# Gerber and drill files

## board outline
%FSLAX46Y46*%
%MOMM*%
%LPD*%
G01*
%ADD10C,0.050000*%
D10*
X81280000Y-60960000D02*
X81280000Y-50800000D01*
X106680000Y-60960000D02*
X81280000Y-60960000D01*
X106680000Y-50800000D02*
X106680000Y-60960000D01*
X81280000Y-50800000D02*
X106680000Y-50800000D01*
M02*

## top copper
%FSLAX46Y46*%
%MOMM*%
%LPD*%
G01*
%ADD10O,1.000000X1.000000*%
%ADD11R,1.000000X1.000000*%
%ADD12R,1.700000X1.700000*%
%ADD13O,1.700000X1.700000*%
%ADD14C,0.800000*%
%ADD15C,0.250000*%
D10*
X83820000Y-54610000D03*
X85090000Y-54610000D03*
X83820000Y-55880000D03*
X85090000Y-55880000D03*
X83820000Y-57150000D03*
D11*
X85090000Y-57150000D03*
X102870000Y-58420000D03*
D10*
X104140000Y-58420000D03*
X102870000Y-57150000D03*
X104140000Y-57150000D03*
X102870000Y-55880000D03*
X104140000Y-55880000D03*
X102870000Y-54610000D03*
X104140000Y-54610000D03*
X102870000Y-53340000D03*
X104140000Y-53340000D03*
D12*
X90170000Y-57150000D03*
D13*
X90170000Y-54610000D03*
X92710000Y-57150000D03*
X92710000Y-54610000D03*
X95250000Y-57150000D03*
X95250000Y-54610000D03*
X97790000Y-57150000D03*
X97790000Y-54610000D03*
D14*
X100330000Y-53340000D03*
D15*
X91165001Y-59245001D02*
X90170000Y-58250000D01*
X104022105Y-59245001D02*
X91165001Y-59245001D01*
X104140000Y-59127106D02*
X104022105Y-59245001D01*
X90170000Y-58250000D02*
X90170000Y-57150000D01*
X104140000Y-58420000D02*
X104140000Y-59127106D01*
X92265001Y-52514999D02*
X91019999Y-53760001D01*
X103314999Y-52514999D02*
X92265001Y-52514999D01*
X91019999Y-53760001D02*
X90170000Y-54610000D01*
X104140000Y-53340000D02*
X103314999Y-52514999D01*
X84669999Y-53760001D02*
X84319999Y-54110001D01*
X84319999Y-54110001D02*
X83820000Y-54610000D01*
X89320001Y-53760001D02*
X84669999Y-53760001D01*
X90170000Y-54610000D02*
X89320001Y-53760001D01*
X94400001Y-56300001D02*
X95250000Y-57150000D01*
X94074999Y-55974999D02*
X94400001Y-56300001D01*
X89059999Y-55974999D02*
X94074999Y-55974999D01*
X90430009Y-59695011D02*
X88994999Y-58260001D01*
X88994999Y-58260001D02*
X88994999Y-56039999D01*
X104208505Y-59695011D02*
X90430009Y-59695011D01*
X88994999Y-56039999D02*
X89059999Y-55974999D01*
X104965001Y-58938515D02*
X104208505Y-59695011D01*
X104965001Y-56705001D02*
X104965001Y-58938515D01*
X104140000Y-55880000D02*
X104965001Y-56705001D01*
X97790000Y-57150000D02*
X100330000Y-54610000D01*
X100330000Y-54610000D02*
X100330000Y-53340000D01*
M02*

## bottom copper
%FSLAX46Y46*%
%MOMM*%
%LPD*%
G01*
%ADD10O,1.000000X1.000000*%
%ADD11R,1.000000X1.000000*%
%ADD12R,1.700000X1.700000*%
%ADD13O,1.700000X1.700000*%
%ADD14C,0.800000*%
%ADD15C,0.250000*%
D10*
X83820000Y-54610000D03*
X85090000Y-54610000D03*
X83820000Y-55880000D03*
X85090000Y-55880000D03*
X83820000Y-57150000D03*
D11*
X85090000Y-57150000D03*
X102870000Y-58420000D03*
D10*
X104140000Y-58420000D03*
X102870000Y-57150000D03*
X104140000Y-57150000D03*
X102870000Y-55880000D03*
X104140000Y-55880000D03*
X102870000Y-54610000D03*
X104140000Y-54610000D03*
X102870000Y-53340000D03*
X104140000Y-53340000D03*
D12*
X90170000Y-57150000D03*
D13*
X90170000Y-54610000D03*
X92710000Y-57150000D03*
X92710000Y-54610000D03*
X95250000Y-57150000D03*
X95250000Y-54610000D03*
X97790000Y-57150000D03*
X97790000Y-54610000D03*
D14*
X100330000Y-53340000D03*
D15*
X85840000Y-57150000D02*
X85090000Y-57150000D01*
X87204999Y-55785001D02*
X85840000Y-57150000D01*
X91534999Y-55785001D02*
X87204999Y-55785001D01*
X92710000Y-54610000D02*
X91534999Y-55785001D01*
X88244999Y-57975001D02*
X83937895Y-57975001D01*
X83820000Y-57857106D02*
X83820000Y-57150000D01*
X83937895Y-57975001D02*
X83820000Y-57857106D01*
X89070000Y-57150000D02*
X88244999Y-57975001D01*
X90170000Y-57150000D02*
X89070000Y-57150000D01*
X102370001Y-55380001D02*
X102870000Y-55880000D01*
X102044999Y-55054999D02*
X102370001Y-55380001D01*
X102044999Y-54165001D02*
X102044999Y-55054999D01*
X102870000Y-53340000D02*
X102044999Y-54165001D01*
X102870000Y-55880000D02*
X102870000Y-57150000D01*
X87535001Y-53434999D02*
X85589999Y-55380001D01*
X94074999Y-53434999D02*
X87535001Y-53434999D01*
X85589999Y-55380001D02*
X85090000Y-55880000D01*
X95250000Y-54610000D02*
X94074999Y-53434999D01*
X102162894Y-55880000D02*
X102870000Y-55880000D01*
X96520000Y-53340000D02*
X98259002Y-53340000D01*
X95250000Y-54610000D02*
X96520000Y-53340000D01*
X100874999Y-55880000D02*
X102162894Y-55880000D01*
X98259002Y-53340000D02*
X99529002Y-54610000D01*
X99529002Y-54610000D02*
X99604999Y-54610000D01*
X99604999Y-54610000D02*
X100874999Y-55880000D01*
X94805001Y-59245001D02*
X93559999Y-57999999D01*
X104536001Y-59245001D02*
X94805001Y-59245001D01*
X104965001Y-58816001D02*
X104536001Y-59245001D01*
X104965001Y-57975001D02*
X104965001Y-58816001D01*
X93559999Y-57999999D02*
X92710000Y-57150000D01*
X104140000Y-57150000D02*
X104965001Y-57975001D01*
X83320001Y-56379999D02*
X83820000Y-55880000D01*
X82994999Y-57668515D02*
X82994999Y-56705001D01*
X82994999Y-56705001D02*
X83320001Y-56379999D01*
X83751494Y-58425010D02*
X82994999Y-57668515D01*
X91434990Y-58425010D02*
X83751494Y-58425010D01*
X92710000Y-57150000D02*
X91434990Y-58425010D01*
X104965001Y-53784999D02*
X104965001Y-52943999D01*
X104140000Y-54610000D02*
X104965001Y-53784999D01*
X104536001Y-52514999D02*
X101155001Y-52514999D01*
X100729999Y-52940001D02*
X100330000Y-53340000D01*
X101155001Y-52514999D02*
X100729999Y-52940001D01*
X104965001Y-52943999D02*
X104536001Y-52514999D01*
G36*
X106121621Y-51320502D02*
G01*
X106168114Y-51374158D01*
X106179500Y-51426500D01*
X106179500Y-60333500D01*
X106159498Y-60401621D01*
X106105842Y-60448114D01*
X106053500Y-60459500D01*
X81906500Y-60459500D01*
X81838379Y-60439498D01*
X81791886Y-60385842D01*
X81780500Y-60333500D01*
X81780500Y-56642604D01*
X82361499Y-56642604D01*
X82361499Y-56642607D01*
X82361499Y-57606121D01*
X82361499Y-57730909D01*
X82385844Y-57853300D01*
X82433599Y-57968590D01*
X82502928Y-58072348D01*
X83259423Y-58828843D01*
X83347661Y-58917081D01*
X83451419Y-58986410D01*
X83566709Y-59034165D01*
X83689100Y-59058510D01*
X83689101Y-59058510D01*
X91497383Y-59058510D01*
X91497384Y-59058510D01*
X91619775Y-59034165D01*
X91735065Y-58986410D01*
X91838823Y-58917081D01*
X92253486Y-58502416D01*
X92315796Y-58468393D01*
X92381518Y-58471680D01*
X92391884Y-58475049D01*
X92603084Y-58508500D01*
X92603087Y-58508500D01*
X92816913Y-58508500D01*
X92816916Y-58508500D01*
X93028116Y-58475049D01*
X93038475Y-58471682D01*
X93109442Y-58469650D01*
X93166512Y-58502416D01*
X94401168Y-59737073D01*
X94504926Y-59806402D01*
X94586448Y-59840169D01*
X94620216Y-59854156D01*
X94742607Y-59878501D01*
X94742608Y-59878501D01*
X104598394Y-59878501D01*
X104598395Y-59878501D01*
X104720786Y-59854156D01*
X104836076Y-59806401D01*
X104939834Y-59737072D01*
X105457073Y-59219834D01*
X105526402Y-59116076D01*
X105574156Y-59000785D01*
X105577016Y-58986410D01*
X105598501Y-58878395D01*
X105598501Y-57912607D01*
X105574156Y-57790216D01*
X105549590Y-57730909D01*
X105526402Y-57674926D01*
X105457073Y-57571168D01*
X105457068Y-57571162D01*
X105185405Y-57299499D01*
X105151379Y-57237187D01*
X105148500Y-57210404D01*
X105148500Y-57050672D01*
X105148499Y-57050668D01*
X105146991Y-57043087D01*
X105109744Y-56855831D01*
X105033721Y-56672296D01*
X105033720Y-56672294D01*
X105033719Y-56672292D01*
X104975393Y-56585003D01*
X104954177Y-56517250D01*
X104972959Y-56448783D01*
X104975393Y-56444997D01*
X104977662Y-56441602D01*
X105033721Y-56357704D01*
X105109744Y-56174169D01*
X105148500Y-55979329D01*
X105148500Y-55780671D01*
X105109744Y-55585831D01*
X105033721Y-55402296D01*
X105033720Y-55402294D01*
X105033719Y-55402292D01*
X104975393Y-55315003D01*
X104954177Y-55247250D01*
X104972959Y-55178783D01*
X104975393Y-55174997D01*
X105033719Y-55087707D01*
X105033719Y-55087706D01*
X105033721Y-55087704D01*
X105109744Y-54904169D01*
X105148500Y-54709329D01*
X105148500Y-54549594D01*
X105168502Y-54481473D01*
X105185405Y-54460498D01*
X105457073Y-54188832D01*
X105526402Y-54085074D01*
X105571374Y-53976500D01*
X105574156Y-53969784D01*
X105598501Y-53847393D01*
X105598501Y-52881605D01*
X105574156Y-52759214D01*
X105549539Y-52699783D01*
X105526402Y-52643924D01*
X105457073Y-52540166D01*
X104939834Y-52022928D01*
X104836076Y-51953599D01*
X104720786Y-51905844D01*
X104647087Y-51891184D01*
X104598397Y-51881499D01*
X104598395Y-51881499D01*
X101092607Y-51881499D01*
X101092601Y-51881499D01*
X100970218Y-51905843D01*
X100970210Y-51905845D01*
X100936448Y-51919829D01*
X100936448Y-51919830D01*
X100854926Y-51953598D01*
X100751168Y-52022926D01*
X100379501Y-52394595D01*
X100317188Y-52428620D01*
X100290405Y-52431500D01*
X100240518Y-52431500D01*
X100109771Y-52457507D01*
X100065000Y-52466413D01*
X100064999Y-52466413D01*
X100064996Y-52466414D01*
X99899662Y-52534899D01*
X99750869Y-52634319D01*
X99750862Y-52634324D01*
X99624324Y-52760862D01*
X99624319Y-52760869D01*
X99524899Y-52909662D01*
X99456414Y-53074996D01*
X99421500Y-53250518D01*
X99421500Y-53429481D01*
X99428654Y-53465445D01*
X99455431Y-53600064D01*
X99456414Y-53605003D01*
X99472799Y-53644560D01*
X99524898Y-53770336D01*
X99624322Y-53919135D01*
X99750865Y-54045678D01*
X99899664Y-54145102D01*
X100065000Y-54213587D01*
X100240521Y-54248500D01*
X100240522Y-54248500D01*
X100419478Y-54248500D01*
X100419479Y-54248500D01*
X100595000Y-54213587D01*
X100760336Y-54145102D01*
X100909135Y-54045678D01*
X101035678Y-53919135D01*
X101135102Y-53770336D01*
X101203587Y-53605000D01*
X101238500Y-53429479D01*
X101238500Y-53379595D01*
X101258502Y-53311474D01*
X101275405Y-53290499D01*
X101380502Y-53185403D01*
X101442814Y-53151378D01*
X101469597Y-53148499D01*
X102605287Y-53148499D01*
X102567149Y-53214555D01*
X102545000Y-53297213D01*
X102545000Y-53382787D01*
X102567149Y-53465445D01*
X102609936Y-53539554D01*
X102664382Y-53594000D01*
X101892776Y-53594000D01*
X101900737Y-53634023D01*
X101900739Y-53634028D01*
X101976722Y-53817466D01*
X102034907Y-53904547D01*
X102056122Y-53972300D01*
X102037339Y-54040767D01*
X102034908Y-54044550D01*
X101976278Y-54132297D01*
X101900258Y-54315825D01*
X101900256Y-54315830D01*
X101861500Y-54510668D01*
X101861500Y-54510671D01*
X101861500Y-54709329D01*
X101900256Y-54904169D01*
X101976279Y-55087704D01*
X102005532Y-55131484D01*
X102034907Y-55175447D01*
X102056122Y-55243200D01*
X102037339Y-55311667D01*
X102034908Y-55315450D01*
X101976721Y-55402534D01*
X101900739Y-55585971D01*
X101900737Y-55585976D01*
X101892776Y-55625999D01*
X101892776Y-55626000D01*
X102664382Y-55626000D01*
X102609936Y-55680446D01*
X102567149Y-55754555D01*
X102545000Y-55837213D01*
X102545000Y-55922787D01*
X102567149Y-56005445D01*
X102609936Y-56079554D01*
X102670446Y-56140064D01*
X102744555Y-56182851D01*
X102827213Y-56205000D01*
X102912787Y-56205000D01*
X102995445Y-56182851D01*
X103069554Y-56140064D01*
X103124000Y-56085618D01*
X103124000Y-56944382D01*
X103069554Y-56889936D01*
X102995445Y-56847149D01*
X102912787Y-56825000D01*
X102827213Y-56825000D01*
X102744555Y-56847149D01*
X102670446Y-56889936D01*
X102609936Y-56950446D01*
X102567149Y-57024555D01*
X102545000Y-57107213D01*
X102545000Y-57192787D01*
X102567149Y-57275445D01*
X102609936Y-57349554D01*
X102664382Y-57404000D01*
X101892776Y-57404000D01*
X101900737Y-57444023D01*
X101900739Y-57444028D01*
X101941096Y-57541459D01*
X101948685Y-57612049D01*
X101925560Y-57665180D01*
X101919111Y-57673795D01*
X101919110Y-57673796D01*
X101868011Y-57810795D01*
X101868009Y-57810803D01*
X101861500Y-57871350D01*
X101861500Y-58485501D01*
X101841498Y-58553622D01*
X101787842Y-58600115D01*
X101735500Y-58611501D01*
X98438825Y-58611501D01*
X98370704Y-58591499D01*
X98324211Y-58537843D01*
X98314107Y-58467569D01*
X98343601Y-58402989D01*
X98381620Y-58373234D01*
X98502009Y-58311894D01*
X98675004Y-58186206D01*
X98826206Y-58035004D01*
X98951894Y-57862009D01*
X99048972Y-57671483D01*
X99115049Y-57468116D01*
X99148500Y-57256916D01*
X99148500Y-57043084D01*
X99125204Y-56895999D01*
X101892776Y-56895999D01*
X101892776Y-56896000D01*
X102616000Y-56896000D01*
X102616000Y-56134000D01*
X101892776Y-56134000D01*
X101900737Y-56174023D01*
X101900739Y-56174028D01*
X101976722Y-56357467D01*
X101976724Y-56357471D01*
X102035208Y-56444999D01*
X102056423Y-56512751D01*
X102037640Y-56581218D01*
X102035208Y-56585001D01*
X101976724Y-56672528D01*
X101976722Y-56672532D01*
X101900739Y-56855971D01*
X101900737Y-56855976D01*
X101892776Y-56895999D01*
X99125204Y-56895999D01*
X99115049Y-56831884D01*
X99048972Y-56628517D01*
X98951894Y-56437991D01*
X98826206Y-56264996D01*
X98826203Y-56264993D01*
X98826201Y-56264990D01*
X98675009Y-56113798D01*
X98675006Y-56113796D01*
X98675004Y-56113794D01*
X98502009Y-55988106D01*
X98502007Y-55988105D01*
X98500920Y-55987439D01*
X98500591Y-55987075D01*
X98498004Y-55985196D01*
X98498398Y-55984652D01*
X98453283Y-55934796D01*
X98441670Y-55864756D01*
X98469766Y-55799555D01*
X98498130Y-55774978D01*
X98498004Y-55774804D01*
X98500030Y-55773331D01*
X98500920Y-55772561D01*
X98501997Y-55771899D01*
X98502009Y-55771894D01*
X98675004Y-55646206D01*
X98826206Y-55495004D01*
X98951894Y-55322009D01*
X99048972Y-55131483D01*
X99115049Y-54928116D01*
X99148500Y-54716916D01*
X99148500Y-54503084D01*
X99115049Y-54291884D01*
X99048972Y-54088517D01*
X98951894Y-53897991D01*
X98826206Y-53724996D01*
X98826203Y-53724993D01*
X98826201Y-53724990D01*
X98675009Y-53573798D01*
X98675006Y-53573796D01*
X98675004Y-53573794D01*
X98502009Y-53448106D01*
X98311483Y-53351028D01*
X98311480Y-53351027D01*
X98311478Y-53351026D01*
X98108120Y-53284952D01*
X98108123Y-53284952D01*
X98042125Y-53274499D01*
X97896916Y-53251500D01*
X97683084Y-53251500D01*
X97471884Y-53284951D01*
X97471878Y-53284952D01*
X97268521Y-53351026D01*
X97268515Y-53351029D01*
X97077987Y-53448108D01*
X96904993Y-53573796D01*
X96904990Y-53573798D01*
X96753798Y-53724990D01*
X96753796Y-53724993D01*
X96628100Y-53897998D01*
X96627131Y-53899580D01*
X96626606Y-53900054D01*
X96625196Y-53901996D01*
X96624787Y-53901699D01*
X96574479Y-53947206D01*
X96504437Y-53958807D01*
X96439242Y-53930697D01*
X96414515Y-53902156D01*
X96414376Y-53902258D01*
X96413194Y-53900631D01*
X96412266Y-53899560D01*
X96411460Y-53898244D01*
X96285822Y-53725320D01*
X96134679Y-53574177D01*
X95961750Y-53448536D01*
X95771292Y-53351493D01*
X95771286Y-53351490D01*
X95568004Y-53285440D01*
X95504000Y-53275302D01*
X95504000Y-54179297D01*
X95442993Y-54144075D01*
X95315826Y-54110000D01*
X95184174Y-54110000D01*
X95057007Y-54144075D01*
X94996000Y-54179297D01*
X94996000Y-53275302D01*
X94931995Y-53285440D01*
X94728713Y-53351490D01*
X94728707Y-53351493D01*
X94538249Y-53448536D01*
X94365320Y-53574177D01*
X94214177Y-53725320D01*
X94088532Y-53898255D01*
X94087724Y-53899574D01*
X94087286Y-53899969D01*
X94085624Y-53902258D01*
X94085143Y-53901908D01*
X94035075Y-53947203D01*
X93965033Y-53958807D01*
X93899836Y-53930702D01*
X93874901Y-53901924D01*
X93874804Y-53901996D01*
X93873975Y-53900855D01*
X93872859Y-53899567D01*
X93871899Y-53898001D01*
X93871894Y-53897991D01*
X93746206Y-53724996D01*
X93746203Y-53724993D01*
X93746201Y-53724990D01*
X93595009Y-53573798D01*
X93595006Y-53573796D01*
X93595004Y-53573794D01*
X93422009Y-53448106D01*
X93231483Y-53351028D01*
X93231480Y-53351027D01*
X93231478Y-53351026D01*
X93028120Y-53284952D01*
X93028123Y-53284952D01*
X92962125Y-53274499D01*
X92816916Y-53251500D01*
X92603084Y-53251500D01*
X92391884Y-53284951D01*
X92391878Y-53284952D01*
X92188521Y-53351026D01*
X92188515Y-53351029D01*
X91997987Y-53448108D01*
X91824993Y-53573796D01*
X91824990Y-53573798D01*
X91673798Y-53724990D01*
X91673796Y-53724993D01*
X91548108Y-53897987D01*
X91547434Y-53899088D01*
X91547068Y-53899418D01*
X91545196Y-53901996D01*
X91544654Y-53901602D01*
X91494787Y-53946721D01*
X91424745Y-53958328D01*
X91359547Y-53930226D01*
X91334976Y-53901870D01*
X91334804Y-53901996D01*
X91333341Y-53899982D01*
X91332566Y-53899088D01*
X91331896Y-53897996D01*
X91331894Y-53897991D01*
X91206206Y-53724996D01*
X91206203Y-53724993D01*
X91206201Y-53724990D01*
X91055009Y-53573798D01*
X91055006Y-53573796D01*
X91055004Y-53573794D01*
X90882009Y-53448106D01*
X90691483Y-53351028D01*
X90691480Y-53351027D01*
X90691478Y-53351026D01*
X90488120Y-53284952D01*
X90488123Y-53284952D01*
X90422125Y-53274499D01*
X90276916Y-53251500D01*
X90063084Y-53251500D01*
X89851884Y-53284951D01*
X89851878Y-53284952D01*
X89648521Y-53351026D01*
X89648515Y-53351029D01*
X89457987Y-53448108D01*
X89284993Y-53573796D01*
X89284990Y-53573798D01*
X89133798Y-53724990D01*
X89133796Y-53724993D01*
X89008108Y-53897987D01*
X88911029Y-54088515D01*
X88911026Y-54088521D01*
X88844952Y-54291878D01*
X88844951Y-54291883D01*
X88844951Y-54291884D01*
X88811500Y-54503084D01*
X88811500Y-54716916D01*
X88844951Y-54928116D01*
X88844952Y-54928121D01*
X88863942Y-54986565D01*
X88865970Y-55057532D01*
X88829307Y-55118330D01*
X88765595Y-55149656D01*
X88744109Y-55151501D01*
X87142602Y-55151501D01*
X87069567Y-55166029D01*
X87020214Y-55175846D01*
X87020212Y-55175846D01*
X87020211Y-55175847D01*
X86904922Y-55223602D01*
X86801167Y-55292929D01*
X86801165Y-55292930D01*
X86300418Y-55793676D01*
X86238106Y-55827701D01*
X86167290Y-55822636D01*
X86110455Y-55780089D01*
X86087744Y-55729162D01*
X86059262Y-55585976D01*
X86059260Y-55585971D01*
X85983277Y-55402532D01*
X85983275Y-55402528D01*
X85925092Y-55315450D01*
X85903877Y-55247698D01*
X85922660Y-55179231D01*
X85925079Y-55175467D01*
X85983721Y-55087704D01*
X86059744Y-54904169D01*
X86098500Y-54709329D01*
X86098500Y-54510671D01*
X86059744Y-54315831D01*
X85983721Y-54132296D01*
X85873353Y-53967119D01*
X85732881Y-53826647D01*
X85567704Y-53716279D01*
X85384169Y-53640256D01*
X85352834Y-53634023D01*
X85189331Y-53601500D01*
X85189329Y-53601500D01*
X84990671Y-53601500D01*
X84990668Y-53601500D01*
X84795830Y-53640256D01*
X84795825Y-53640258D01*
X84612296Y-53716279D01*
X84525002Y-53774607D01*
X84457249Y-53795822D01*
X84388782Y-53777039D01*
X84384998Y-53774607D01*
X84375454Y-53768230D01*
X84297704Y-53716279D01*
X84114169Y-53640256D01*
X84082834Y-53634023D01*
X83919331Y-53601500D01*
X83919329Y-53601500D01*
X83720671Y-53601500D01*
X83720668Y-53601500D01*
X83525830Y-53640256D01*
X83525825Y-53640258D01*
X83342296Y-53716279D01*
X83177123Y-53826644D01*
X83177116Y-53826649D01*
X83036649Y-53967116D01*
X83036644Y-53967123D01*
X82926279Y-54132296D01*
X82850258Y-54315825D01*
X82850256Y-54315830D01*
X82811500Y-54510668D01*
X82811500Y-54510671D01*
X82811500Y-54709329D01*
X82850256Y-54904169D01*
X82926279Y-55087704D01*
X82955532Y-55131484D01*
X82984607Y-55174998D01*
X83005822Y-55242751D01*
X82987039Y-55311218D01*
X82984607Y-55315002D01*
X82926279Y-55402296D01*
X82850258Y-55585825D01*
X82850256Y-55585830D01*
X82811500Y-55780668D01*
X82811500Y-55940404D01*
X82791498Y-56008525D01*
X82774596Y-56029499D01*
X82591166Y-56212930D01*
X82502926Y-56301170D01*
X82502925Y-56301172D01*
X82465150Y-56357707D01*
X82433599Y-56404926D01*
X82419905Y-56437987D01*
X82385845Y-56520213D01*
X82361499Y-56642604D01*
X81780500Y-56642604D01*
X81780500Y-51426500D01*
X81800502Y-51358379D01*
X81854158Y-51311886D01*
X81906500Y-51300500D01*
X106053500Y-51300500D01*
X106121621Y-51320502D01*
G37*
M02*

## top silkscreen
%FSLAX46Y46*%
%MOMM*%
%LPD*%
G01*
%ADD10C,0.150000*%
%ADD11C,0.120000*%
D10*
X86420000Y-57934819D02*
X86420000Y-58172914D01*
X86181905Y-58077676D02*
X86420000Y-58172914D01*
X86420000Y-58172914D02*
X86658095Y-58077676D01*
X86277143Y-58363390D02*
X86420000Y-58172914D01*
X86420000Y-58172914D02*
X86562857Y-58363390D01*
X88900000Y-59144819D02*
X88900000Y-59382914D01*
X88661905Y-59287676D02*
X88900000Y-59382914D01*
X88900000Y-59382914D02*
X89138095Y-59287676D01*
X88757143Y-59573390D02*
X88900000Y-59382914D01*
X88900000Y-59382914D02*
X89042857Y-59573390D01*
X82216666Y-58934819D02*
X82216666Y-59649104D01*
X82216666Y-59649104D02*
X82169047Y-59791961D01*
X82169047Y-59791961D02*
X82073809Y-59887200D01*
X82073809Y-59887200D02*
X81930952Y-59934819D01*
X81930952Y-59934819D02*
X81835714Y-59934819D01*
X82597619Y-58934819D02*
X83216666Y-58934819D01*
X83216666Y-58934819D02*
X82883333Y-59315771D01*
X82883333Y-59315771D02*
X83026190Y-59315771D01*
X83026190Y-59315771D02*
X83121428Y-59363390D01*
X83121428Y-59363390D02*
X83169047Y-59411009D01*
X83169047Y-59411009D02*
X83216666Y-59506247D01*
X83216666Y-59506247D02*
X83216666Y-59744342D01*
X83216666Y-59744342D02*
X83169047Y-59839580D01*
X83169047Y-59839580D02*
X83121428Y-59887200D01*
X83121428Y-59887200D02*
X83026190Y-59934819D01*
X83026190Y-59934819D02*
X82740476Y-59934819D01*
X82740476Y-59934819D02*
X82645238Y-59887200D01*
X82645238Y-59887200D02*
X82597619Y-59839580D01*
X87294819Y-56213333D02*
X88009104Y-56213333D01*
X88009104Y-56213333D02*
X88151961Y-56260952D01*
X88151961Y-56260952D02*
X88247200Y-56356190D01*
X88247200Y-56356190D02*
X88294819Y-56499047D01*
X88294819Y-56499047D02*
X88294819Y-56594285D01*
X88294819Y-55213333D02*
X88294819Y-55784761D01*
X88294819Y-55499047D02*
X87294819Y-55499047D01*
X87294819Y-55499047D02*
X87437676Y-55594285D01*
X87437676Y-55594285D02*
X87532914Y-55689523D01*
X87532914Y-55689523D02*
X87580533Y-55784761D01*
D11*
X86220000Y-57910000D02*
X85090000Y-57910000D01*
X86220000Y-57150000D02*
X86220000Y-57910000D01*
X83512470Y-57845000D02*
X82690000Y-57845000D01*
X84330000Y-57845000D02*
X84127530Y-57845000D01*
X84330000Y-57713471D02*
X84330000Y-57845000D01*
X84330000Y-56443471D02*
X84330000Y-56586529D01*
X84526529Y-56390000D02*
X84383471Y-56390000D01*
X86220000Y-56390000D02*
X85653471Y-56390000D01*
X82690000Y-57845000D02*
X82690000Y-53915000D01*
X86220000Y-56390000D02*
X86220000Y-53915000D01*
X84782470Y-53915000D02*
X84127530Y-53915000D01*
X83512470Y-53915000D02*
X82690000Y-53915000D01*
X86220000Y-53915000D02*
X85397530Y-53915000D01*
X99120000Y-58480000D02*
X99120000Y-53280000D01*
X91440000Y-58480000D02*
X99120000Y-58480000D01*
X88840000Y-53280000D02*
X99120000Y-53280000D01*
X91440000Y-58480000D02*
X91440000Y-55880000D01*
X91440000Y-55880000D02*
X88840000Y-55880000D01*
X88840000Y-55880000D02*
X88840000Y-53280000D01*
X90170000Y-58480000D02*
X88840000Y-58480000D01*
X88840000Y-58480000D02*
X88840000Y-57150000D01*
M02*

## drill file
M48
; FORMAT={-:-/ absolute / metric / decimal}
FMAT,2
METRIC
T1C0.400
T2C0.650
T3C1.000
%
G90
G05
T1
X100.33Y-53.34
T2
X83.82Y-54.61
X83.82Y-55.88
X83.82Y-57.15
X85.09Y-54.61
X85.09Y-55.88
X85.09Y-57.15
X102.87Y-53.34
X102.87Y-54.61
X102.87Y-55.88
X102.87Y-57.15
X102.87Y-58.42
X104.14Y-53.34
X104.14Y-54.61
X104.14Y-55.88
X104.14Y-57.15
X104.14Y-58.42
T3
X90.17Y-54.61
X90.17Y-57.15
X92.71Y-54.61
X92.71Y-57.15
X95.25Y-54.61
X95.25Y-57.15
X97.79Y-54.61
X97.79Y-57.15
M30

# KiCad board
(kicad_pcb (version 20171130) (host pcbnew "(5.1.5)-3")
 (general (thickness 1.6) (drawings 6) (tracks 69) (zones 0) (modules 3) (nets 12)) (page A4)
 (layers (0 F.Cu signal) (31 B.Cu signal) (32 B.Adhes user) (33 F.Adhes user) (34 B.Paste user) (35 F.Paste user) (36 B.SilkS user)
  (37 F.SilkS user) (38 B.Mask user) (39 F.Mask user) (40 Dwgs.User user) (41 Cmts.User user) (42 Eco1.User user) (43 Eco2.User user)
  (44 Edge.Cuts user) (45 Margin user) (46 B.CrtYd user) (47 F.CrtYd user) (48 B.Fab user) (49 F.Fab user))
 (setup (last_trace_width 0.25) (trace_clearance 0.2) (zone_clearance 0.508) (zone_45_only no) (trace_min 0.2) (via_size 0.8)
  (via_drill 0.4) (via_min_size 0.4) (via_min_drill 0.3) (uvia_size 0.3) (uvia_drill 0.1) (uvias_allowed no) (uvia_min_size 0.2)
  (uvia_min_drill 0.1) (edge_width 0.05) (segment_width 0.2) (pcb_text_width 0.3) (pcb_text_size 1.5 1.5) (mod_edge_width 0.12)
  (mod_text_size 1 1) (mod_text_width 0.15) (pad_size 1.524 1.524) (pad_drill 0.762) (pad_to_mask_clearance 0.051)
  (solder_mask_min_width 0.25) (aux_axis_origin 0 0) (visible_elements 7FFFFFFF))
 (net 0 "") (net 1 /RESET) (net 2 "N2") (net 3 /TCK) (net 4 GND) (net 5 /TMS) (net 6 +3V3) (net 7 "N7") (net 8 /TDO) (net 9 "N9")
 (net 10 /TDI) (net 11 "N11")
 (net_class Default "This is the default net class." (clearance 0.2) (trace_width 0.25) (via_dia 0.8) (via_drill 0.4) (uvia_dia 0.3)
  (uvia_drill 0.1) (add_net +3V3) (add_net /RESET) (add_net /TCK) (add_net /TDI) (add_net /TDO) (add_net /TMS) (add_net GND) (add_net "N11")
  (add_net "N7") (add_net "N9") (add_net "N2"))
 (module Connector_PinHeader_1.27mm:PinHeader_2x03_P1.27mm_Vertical (layer F.Cu) (at 85.09 57.15 180)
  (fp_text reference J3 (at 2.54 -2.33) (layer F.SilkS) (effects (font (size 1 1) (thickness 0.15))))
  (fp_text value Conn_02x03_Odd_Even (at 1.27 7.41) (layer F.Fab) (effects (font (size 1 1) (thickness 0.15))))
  (fp_line (start -1.13 -0.76) (end 0 -0.76) (layer F.SilkS) (width 0.12))
  (fp_line (start -1.13 0) (end -1.13 -0.76) (layer F.SilkS) (width 0.12))
  (fp_line (start 1.57753 -0.695) (end 2.4 -0.695) (layer F.SilkS) (width 0.12))
  (fp_line (start 0.76 -0.695) (end 0.96247 -0.695) (layer F.SilkS) (width 0.12))
  (fp_line (start 0.76 -0.563471) (end 0.76 -0.695) (layer F.SilkS) (width 0.12))
  (fp_line (start 0.76 0.706529) (end 0.76 0.563471) (layer F.SilkS) (width 0.12))
  (fp_line (start 0.563471 0.76) (end 0.706529 0.76) (layer F.SilkS) (width 0.12))
  (fp_line (start -1.13 0.76) (end -0.563471 0.76) (layer F.SilkS) (width 0.12))
  (fp_line (start 2.4 -0.695) (end 2.4 3.235) (layer F.SilkS) (width 0.12))
  (fp_line (start -1.13 0.76) (end -1.13 3.235) (layer F.SilkS) (width 0.12))
  (fp_line (start 0.30753 3.235) (end 0.96247 3.235) (layer F.SilkS) (width 0.12))
  (fp_line (start 1.57753 3.235) (end 2.4 3.235) (layer F.SilkS) (width 0.12))
  (fp_line (start -1.13 3.235) (end -0.30753 3.235) (layer F.SilkS) (width 0.12))
  (pad 6 thru_hole oval (at 1.27 2.54 180) (size 1 1) (drill 0.65) (layers *.Cu *.Mask) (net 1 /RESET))
  (pad 5 thru_hole oval (at 0 2.54 180) (size 1 1) (drill 0.65) (layers *.Cu *.Mask) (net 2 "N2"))
  (pad 4 thru_hole oval (at 1.27 1.27 180) (size 1 1) (drill 0.65) (layers *.Cu *.Mask) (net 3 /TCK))
  (pad 3 thru_hole oval (at 0 1.27 180) (size 1 1) (drill 0.65) (layers *.Cu *.Mask) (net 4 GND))
  (pad 2 thru_hole oval (at 1.27 0 180) (size 1 1) (drill 0.65) (layers *.Cu *.Mask) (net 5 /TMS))
  (pad 1 thru_hole rect (at 0 0 180) (size 1 1) (drill 0.65) (layers *.Cu *.Mask) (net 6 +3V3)))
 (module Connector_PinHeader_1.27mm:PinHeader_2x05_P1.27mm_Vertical (layer B.Cu) (at 102.87 58.42)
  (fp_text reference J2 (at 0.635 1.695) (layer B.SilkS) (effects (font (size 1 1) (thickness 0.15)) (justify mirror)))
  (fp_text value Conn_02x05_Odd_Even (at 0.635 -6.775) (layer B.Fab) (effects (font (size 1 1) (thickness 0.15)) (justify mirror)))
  (pad 1 thru_hole rect (at 0 0) (size 1 1) (drill 0.65) (layers *.Cu *.Mask) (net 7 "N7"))
  (pad 2 thru_hole oval (at 1.27 0) (size 1 1) (drill 0.65) (layers *.Cu *.Mask) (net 5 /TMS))
  (pad 3 thru_hole oval (at 0 -1.27) (size 1 1) (drill 0.65) (layers *.Cu *.Mask) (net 4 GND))
  (pad 4 thru_hole oval (at 1.27 -1.27) (size 1 1) (drill 0.65) (layers *.Cu *.Mask) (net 3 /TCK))
  (pad 5 thru_hole oval (at 0 -2.54) (size 1 1) (drill 0.65) (layers *.Cu *.Mask) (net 4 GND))
  (pad 6 thru_hole oval (at 1.27 -2.54) (size 1 1) (drill 0.65) (layers *.Cu *.Mask) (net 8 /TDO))
  (pad 7 thru_hole oval (at 0 -3.81) (size 1 1) (drill 0.65) (layers *.Cu *.Mask) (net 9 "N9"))
  (pad 8 thru_hole oval (at 1.27 -3.81) (size 1 1) (drill 0.65) (layers *.Cu *.Mask) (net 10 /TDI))
  (pad 9 thru_hole oval (at 0 -5.08) (size 1 1) (drill 0.65) (layers *.Cu *.Mask) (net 4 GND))
  (pad 10 thru_hole oval (at 1.27 -5.08) (size 1 1) (drill 0.65) (layers *.Cu *.Mask) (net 1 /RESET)))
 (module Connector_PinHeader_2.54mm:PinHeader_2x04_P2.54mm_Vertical (layer F.Cu) (at 90.17 57.15 90)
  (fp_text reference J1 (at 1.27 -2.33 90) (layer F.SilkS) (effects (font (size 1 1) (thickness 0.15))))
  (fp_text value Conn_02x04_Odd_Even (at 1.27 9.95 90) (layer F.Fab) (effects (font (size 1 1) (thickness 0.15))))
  (fp_line (start -1.33 8.95) (end 3.87 8.95) (layer F.SilkS) (width 0.12))
  (fp_line (start -1.33 1.27) (end -1.33 8.95) (layer F.SilkS) (width 0.12))
  (fp_line (start 3.87 -1.33) (end 3.87 8.95) (layer F.SilkS) (width 0.12))
  (fp_line (start -1.33 1.27) (end 1.27 1.27) (layer F.SilkS) (width 0.12))
  (fp_line (start 1.27 1.27) (end 1.27 -1.33) (layer F.SilkS) (width 0.12))
  (fp_line (start 1.27 -1.33) (end 3.87 -1.33) (layer F.SilkS) (width 0.12))
  (fp_line (start -1.33 0) (end -1.33 -1.33) (layer F.SilkS) (width 0.12))
  (fp_line (start -1.33 -1.33) (end 0 -1.33) (layer F.SilkS) (width 0.12))
  (pad 1 thru_hole rect (at 0 0 90) (size 1.7 1.7) (drill 1) (layers *.Cu *.Mask) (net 5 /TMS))
  (pad 2 thru_hole oval (at 2.54 0 90) (size 1.7 1.7) (drill 1) (layers *.Cu *.Mask) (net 1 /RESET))
  (pad 3 thru_hole oval (at 0 2.54 90) (size 1.7 1.7) (drill 1) (layers *.Cu *.Mask) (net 3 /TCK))
  (pad 4 thru_hole oval (at 2.54 2.54 90) (size 1.7 1.7) (drill 1) (layers *.Cu *.Mask) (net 6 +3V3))
  (pad 5 thru_hole oval (at 0 5.08 90) (size 1.7 1.7) (drill 1) (layers *.Cu *.Mask) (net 8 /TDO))
  (pad 6 thru_hole oval (at 2.54 5.08 90) (size 1.7 1.7) (drill 1) (layers *.Cu *.Mask) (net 4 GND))
  (pad 7 thru_hole oval (at 0 7.62 90) (size 1.7 1.7) (drill 1) (layers *.Cu *.Mask) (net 10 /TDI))
  (pad 8 thru_hole oval (at 2.54 7.62 90) (size 1.7 1.7) (drill 1) (layers *.Cu *.Mask) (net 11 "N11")))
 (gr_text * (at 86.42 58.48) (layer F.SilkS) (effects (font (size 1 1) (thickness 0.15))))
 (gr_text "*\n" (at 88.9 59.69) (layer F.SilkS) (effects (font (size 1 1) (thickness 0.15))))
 (gr_line (start 81.28 60.96) (end 81.28 50.8) (layer Edge.Cuts) (width 0.05))
 (gr_line (start 106.68 60.96) (end 81.28 60.96) (layer Edge.Cuts) (width 0.05))
 (gr_line (start 106.68 50.8) (end 106.68 60.96) (layer Edge.Cuts) (width 0.05))
 (gr_line (start 81.28 50.8) (end 106.68 50.8) (layer Edge.Cuts) (width 0.05))
 (segment (start 85.84 57.15) (end 85.09 57.15) (width 0.25) (layer B.Cu) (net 6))
 (segment (start 87.204999 55.785001) (end 85.84 57.15) (width 0.25) (layer B.Cu) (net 6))
 (segment (start 91.534999 55.785001) (end 87.204999 55.785001) (width 0.25) (layer B.Cu) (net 6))
 (segment (start 92.71 54.61) (end 91.534999 55.785001) (width 0.25) (layer B.Cu) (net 6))
 (segment (start 88.244999 57.975001) (end 83.937895 57.975001) (width 0.25) (layer B.Cu) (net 5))
 (segment (start 83.82 57.857106) (end 83.82 57.15) (width 0.25) (layer B.Cu) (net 5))
 (segment (start 83.937895 57.975001) (end 83.82 57.857106) (width 0.25) (layer B.Cu) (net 5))
 (segment (start 89.07 57.15) (end 88.244999 57.975001) (width 0.25) (layer B.Cu) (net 5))
 (segment (start 90.17 57.15) (end 89.07 57.15) (width 0.25) (layer B.Cu) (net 5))
 (segment (start 91.165001 59.245001) (end 90.17 58.25) (width 0.25) (layer F.Cu) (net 5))
 (segment (start 104.022105 59.245001) (end 91.165001 59.245001) (width 0.25) (layer F.Cu) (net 5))
 (segment (start 104.14 59.127106) (end 104.022105 59.245001) (width 0.25) (layer F.Cu) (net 5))
 (segment (start 90.17 58.25) (end 90.17 57.15) (width 0.25) (layer F.Cu) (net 5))
 (segment (start 104.14 58.42) (end 104.14 59.127106) (width 0.25) (layer F.Cu) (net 5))
 (segment (start 102.370001 55.380001) (end 102.87 55.88) (width 0.25) (layer B.Cu) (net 4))
 (segment (start 102.044999 55.054999) (end 102.370001 55.380001) (width 0.25) (layer B.Cu) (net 4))
 (segment (start 102.044999 54.165001) (end 102.044999 55.054999) (width 0.25) (layer B.Cu) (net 4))
 (segment (start 102.87 53.34) (end 102.044999 54.165001) (width 0.25) (layer B.Cu) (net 4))
 (segment (start 102.87 55.88) (end 102.87 57.15) (width 0.25) (layer B.Cu) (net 4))
 (segment (start 87.535001 53.434999) (end 85.589999 55.380001) (width 0.25) (layer B.Cu) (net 4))
 (segment (start 94.074999 53.434999) (end 87.535001 53.434999) (width 0.25) (layer B.Cu) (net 4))
 (segment (start 85.589999 55.380001) (end 85.09 55.88) (width 0.25) (layer B.Cu) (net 4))
 (segment (start 95.25 54.61) (end 94.074999 53.434999) (width 0.25) (layer B.Cu) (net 4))
 (segment (start 102.162894 55.88) (end 102.87 55.88) (width 0.25) (layer B.Cu) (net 4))
 (segment (start 96.52 53.34) (end 98.259002 53.34) (width 0.25) (layer B.Cu) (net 4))
 (segment (start 95.25 54.61) (end 96.52 53.34) (width 0.25) (layer B.Cu) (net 4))
 (segment (start 100.874999 55.88) (end 102.162894 55.88) (width 0.25) (layer B.Cu) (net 4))
 (segment (start 98.259002 53.34) (end 99.529002 54.61) (width 0.25) (layer B.Cu) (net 4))
 (segment (start 99.529002 54.61) (end 99.604999 54.61) (width 0.25) (layer B.Cu) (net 4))
 (segment (start 99.604999 54.61) (end 100.874999 55.88) (width 0.25) (layer B.Cu) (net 4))
 (segment (start 94.805001 59.245001) (end 93.559999 57.999999) (width 0.25) (layer B.Cu) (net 3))
 (segment (start 104.536001 59.245001) (end 94.805001 59.245001) (width 0.25) (layer B.Cu) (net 3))
 (segment (start 104.965001 58.816001) (end 104.536001 59.245001) (width 0.25) (layer B.Cu) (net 3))
 (segment (start 104.965001 57.975001) (end 104.965001 58.816001) (width 0.25) (layer B.Cu) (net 3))
 (segment (start 93.559999 57.999999) (end 92.71 57.15) (width 0.25) (layer B.Cu) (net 3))
 (segment (start 104.14 57.15) (end 104.965001 57.975001) (width 0.25) (layer B.Cu) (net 3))
 (segment (start 83.320001 56.379999) (end 83.82 55.88) (width 0.25) (layer B.Cu) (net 3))
 (segment (start 82.994999 57.668515) (end 82.994999 56.705001) (width 0.25) (layer B.Cu) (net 3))
 (segment (start 82.994999 56.705001) (end 83.320001 56.379999) (width 0.25) (layer B.Cu) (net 3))
 (segment (start 83.751494 58.42501) (end 82.994999 57.668515) (width 0.25) (layer B.Cu) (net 3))
 (segment (start 91.43499 58.42501) (end 83.751494 58.42501) (width 0.25) (layer B.Cu) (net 3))
 (segment (start 92.71 57.15) (end 91.43499 58.42501) (width 0.25) (layer B.Cu) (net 3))
 (segment (start 92.265001 52.514999) (end 91.019999 53.760001) (width 0.25) (layer F.Cu) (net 1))
 (segment (start 103.314999 52.514999) (end 92.265001 52.514999) (width 0.25) (layer F.Cu) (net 1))
 (segment (start 91.019999 53.760001) (end 90.17 54.61) (width 0.25) (layer F.Cu) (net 1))
 (segment (start 104.14 53.34) (end 103.314999 52.514999) (width 0.25) (layer F.Cu) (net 1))
 (segment (start 84.669999 53.760001) (end 84.319999 54.110001) (width 0.25) (layer F.Cu) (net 1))
 (segment (start 84.319999 54.110001) (end 83.82 54.61) (width 0.25) (layer F.Cu) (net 1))
 (segment (start 89.320001 53.760001) (end 84.669999 53.760001) (width 0.25) (layer F.Cu) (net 1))
 (segment (start 90.17 54.61) (end 89.320001 53.760001) (width 0.25) (layer F.Cu) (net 1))
 (segment (start 94.400001 56.300001) (end 95.25 57.15) (width 0.25) (layer F.Cu) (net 8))
 (segment (start 94.074999 55.974999) (end 94.400001 56.300001) (width 0.25) (layer F.Cu) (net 8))
 (segment (start 89.059999 55.974999) (end 94.074999 55.974999) (width 0.25) (layer F.Cu) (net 8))
 (segment (start 90.430009 59.695011) (end 88.994999 58.260001) (width 0.25) (layer F.Cu) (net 8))
 (segment (start 88.994999 58.260001) (end 88.994999 56.039999) (width 0.25) (layer F.Cu) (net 8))
 (segment (start 104.208505 59.695011) (end 90.430009 59.695011) (width 0.25) (layer F.Cu) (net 8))
 (segment (start 88.994999 56.039999) (end 89.059999 55.974999) (width 0.25) (layer F.Cu) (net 8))
 (segment (start 104.965001 58.938515) (end 104.208505 59.695011) (width 0.25) (layer F.Cu) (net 8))
 (segment (start 104.965001 56.705001) (end 104.965001 58.938515) (width 0.25) (layer F.Cu) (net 8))
 (segment (start 104.14 55.88) (end 104.965001 56.705001) (width 0.25) (layer F.Cu) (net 8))
 (segment (start 97.79 57.15) (end 100.33 54.61) (width 0.25) (layer F.Cu) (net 10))
 (segment (start 104.965001 53.784999) (end 104.965001 52.943999) (width 0.25) (layer B.Cu) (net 10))
 (segment (start 104.14 54.61) (end 104.965001 53.784999) (width 0.25) (layer B.Cu) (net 10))
 (segment (start 104.536001 52.514999) (end 101.155001 52.514999) (width 0.25) (layer B.Cu) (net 10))
 (segment (start 100.729999 52.940001) (end 100.33 53.34) (width 0.25) (layer B.Cu) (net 10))
 (segment (start 101.155001 52.514999) (end 100.729999 52.940001) (width 0.25) (layer B.Cu) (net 10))
 (segment (start 104.965001 52.943999) (end 104.536001 52.514999) (width 0.25) (layer B.Cu) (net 10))
 (via (at 100.33 53.34) (size 0.8) (drill 0.4) (layers F.Cu B.Cu) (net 10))
 (segment (start 100.33 54.61) (end 100.33 53.34) (width 0.25) (layer F.Cu) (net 10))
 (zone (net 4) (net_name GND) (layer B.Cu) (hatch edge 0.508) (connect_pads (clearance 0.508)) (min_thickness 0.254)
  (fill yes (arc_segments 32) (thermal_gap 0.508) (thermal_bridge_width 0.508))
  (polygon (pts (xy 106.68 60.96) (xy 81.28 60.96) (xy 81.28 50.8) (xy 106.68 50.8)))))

